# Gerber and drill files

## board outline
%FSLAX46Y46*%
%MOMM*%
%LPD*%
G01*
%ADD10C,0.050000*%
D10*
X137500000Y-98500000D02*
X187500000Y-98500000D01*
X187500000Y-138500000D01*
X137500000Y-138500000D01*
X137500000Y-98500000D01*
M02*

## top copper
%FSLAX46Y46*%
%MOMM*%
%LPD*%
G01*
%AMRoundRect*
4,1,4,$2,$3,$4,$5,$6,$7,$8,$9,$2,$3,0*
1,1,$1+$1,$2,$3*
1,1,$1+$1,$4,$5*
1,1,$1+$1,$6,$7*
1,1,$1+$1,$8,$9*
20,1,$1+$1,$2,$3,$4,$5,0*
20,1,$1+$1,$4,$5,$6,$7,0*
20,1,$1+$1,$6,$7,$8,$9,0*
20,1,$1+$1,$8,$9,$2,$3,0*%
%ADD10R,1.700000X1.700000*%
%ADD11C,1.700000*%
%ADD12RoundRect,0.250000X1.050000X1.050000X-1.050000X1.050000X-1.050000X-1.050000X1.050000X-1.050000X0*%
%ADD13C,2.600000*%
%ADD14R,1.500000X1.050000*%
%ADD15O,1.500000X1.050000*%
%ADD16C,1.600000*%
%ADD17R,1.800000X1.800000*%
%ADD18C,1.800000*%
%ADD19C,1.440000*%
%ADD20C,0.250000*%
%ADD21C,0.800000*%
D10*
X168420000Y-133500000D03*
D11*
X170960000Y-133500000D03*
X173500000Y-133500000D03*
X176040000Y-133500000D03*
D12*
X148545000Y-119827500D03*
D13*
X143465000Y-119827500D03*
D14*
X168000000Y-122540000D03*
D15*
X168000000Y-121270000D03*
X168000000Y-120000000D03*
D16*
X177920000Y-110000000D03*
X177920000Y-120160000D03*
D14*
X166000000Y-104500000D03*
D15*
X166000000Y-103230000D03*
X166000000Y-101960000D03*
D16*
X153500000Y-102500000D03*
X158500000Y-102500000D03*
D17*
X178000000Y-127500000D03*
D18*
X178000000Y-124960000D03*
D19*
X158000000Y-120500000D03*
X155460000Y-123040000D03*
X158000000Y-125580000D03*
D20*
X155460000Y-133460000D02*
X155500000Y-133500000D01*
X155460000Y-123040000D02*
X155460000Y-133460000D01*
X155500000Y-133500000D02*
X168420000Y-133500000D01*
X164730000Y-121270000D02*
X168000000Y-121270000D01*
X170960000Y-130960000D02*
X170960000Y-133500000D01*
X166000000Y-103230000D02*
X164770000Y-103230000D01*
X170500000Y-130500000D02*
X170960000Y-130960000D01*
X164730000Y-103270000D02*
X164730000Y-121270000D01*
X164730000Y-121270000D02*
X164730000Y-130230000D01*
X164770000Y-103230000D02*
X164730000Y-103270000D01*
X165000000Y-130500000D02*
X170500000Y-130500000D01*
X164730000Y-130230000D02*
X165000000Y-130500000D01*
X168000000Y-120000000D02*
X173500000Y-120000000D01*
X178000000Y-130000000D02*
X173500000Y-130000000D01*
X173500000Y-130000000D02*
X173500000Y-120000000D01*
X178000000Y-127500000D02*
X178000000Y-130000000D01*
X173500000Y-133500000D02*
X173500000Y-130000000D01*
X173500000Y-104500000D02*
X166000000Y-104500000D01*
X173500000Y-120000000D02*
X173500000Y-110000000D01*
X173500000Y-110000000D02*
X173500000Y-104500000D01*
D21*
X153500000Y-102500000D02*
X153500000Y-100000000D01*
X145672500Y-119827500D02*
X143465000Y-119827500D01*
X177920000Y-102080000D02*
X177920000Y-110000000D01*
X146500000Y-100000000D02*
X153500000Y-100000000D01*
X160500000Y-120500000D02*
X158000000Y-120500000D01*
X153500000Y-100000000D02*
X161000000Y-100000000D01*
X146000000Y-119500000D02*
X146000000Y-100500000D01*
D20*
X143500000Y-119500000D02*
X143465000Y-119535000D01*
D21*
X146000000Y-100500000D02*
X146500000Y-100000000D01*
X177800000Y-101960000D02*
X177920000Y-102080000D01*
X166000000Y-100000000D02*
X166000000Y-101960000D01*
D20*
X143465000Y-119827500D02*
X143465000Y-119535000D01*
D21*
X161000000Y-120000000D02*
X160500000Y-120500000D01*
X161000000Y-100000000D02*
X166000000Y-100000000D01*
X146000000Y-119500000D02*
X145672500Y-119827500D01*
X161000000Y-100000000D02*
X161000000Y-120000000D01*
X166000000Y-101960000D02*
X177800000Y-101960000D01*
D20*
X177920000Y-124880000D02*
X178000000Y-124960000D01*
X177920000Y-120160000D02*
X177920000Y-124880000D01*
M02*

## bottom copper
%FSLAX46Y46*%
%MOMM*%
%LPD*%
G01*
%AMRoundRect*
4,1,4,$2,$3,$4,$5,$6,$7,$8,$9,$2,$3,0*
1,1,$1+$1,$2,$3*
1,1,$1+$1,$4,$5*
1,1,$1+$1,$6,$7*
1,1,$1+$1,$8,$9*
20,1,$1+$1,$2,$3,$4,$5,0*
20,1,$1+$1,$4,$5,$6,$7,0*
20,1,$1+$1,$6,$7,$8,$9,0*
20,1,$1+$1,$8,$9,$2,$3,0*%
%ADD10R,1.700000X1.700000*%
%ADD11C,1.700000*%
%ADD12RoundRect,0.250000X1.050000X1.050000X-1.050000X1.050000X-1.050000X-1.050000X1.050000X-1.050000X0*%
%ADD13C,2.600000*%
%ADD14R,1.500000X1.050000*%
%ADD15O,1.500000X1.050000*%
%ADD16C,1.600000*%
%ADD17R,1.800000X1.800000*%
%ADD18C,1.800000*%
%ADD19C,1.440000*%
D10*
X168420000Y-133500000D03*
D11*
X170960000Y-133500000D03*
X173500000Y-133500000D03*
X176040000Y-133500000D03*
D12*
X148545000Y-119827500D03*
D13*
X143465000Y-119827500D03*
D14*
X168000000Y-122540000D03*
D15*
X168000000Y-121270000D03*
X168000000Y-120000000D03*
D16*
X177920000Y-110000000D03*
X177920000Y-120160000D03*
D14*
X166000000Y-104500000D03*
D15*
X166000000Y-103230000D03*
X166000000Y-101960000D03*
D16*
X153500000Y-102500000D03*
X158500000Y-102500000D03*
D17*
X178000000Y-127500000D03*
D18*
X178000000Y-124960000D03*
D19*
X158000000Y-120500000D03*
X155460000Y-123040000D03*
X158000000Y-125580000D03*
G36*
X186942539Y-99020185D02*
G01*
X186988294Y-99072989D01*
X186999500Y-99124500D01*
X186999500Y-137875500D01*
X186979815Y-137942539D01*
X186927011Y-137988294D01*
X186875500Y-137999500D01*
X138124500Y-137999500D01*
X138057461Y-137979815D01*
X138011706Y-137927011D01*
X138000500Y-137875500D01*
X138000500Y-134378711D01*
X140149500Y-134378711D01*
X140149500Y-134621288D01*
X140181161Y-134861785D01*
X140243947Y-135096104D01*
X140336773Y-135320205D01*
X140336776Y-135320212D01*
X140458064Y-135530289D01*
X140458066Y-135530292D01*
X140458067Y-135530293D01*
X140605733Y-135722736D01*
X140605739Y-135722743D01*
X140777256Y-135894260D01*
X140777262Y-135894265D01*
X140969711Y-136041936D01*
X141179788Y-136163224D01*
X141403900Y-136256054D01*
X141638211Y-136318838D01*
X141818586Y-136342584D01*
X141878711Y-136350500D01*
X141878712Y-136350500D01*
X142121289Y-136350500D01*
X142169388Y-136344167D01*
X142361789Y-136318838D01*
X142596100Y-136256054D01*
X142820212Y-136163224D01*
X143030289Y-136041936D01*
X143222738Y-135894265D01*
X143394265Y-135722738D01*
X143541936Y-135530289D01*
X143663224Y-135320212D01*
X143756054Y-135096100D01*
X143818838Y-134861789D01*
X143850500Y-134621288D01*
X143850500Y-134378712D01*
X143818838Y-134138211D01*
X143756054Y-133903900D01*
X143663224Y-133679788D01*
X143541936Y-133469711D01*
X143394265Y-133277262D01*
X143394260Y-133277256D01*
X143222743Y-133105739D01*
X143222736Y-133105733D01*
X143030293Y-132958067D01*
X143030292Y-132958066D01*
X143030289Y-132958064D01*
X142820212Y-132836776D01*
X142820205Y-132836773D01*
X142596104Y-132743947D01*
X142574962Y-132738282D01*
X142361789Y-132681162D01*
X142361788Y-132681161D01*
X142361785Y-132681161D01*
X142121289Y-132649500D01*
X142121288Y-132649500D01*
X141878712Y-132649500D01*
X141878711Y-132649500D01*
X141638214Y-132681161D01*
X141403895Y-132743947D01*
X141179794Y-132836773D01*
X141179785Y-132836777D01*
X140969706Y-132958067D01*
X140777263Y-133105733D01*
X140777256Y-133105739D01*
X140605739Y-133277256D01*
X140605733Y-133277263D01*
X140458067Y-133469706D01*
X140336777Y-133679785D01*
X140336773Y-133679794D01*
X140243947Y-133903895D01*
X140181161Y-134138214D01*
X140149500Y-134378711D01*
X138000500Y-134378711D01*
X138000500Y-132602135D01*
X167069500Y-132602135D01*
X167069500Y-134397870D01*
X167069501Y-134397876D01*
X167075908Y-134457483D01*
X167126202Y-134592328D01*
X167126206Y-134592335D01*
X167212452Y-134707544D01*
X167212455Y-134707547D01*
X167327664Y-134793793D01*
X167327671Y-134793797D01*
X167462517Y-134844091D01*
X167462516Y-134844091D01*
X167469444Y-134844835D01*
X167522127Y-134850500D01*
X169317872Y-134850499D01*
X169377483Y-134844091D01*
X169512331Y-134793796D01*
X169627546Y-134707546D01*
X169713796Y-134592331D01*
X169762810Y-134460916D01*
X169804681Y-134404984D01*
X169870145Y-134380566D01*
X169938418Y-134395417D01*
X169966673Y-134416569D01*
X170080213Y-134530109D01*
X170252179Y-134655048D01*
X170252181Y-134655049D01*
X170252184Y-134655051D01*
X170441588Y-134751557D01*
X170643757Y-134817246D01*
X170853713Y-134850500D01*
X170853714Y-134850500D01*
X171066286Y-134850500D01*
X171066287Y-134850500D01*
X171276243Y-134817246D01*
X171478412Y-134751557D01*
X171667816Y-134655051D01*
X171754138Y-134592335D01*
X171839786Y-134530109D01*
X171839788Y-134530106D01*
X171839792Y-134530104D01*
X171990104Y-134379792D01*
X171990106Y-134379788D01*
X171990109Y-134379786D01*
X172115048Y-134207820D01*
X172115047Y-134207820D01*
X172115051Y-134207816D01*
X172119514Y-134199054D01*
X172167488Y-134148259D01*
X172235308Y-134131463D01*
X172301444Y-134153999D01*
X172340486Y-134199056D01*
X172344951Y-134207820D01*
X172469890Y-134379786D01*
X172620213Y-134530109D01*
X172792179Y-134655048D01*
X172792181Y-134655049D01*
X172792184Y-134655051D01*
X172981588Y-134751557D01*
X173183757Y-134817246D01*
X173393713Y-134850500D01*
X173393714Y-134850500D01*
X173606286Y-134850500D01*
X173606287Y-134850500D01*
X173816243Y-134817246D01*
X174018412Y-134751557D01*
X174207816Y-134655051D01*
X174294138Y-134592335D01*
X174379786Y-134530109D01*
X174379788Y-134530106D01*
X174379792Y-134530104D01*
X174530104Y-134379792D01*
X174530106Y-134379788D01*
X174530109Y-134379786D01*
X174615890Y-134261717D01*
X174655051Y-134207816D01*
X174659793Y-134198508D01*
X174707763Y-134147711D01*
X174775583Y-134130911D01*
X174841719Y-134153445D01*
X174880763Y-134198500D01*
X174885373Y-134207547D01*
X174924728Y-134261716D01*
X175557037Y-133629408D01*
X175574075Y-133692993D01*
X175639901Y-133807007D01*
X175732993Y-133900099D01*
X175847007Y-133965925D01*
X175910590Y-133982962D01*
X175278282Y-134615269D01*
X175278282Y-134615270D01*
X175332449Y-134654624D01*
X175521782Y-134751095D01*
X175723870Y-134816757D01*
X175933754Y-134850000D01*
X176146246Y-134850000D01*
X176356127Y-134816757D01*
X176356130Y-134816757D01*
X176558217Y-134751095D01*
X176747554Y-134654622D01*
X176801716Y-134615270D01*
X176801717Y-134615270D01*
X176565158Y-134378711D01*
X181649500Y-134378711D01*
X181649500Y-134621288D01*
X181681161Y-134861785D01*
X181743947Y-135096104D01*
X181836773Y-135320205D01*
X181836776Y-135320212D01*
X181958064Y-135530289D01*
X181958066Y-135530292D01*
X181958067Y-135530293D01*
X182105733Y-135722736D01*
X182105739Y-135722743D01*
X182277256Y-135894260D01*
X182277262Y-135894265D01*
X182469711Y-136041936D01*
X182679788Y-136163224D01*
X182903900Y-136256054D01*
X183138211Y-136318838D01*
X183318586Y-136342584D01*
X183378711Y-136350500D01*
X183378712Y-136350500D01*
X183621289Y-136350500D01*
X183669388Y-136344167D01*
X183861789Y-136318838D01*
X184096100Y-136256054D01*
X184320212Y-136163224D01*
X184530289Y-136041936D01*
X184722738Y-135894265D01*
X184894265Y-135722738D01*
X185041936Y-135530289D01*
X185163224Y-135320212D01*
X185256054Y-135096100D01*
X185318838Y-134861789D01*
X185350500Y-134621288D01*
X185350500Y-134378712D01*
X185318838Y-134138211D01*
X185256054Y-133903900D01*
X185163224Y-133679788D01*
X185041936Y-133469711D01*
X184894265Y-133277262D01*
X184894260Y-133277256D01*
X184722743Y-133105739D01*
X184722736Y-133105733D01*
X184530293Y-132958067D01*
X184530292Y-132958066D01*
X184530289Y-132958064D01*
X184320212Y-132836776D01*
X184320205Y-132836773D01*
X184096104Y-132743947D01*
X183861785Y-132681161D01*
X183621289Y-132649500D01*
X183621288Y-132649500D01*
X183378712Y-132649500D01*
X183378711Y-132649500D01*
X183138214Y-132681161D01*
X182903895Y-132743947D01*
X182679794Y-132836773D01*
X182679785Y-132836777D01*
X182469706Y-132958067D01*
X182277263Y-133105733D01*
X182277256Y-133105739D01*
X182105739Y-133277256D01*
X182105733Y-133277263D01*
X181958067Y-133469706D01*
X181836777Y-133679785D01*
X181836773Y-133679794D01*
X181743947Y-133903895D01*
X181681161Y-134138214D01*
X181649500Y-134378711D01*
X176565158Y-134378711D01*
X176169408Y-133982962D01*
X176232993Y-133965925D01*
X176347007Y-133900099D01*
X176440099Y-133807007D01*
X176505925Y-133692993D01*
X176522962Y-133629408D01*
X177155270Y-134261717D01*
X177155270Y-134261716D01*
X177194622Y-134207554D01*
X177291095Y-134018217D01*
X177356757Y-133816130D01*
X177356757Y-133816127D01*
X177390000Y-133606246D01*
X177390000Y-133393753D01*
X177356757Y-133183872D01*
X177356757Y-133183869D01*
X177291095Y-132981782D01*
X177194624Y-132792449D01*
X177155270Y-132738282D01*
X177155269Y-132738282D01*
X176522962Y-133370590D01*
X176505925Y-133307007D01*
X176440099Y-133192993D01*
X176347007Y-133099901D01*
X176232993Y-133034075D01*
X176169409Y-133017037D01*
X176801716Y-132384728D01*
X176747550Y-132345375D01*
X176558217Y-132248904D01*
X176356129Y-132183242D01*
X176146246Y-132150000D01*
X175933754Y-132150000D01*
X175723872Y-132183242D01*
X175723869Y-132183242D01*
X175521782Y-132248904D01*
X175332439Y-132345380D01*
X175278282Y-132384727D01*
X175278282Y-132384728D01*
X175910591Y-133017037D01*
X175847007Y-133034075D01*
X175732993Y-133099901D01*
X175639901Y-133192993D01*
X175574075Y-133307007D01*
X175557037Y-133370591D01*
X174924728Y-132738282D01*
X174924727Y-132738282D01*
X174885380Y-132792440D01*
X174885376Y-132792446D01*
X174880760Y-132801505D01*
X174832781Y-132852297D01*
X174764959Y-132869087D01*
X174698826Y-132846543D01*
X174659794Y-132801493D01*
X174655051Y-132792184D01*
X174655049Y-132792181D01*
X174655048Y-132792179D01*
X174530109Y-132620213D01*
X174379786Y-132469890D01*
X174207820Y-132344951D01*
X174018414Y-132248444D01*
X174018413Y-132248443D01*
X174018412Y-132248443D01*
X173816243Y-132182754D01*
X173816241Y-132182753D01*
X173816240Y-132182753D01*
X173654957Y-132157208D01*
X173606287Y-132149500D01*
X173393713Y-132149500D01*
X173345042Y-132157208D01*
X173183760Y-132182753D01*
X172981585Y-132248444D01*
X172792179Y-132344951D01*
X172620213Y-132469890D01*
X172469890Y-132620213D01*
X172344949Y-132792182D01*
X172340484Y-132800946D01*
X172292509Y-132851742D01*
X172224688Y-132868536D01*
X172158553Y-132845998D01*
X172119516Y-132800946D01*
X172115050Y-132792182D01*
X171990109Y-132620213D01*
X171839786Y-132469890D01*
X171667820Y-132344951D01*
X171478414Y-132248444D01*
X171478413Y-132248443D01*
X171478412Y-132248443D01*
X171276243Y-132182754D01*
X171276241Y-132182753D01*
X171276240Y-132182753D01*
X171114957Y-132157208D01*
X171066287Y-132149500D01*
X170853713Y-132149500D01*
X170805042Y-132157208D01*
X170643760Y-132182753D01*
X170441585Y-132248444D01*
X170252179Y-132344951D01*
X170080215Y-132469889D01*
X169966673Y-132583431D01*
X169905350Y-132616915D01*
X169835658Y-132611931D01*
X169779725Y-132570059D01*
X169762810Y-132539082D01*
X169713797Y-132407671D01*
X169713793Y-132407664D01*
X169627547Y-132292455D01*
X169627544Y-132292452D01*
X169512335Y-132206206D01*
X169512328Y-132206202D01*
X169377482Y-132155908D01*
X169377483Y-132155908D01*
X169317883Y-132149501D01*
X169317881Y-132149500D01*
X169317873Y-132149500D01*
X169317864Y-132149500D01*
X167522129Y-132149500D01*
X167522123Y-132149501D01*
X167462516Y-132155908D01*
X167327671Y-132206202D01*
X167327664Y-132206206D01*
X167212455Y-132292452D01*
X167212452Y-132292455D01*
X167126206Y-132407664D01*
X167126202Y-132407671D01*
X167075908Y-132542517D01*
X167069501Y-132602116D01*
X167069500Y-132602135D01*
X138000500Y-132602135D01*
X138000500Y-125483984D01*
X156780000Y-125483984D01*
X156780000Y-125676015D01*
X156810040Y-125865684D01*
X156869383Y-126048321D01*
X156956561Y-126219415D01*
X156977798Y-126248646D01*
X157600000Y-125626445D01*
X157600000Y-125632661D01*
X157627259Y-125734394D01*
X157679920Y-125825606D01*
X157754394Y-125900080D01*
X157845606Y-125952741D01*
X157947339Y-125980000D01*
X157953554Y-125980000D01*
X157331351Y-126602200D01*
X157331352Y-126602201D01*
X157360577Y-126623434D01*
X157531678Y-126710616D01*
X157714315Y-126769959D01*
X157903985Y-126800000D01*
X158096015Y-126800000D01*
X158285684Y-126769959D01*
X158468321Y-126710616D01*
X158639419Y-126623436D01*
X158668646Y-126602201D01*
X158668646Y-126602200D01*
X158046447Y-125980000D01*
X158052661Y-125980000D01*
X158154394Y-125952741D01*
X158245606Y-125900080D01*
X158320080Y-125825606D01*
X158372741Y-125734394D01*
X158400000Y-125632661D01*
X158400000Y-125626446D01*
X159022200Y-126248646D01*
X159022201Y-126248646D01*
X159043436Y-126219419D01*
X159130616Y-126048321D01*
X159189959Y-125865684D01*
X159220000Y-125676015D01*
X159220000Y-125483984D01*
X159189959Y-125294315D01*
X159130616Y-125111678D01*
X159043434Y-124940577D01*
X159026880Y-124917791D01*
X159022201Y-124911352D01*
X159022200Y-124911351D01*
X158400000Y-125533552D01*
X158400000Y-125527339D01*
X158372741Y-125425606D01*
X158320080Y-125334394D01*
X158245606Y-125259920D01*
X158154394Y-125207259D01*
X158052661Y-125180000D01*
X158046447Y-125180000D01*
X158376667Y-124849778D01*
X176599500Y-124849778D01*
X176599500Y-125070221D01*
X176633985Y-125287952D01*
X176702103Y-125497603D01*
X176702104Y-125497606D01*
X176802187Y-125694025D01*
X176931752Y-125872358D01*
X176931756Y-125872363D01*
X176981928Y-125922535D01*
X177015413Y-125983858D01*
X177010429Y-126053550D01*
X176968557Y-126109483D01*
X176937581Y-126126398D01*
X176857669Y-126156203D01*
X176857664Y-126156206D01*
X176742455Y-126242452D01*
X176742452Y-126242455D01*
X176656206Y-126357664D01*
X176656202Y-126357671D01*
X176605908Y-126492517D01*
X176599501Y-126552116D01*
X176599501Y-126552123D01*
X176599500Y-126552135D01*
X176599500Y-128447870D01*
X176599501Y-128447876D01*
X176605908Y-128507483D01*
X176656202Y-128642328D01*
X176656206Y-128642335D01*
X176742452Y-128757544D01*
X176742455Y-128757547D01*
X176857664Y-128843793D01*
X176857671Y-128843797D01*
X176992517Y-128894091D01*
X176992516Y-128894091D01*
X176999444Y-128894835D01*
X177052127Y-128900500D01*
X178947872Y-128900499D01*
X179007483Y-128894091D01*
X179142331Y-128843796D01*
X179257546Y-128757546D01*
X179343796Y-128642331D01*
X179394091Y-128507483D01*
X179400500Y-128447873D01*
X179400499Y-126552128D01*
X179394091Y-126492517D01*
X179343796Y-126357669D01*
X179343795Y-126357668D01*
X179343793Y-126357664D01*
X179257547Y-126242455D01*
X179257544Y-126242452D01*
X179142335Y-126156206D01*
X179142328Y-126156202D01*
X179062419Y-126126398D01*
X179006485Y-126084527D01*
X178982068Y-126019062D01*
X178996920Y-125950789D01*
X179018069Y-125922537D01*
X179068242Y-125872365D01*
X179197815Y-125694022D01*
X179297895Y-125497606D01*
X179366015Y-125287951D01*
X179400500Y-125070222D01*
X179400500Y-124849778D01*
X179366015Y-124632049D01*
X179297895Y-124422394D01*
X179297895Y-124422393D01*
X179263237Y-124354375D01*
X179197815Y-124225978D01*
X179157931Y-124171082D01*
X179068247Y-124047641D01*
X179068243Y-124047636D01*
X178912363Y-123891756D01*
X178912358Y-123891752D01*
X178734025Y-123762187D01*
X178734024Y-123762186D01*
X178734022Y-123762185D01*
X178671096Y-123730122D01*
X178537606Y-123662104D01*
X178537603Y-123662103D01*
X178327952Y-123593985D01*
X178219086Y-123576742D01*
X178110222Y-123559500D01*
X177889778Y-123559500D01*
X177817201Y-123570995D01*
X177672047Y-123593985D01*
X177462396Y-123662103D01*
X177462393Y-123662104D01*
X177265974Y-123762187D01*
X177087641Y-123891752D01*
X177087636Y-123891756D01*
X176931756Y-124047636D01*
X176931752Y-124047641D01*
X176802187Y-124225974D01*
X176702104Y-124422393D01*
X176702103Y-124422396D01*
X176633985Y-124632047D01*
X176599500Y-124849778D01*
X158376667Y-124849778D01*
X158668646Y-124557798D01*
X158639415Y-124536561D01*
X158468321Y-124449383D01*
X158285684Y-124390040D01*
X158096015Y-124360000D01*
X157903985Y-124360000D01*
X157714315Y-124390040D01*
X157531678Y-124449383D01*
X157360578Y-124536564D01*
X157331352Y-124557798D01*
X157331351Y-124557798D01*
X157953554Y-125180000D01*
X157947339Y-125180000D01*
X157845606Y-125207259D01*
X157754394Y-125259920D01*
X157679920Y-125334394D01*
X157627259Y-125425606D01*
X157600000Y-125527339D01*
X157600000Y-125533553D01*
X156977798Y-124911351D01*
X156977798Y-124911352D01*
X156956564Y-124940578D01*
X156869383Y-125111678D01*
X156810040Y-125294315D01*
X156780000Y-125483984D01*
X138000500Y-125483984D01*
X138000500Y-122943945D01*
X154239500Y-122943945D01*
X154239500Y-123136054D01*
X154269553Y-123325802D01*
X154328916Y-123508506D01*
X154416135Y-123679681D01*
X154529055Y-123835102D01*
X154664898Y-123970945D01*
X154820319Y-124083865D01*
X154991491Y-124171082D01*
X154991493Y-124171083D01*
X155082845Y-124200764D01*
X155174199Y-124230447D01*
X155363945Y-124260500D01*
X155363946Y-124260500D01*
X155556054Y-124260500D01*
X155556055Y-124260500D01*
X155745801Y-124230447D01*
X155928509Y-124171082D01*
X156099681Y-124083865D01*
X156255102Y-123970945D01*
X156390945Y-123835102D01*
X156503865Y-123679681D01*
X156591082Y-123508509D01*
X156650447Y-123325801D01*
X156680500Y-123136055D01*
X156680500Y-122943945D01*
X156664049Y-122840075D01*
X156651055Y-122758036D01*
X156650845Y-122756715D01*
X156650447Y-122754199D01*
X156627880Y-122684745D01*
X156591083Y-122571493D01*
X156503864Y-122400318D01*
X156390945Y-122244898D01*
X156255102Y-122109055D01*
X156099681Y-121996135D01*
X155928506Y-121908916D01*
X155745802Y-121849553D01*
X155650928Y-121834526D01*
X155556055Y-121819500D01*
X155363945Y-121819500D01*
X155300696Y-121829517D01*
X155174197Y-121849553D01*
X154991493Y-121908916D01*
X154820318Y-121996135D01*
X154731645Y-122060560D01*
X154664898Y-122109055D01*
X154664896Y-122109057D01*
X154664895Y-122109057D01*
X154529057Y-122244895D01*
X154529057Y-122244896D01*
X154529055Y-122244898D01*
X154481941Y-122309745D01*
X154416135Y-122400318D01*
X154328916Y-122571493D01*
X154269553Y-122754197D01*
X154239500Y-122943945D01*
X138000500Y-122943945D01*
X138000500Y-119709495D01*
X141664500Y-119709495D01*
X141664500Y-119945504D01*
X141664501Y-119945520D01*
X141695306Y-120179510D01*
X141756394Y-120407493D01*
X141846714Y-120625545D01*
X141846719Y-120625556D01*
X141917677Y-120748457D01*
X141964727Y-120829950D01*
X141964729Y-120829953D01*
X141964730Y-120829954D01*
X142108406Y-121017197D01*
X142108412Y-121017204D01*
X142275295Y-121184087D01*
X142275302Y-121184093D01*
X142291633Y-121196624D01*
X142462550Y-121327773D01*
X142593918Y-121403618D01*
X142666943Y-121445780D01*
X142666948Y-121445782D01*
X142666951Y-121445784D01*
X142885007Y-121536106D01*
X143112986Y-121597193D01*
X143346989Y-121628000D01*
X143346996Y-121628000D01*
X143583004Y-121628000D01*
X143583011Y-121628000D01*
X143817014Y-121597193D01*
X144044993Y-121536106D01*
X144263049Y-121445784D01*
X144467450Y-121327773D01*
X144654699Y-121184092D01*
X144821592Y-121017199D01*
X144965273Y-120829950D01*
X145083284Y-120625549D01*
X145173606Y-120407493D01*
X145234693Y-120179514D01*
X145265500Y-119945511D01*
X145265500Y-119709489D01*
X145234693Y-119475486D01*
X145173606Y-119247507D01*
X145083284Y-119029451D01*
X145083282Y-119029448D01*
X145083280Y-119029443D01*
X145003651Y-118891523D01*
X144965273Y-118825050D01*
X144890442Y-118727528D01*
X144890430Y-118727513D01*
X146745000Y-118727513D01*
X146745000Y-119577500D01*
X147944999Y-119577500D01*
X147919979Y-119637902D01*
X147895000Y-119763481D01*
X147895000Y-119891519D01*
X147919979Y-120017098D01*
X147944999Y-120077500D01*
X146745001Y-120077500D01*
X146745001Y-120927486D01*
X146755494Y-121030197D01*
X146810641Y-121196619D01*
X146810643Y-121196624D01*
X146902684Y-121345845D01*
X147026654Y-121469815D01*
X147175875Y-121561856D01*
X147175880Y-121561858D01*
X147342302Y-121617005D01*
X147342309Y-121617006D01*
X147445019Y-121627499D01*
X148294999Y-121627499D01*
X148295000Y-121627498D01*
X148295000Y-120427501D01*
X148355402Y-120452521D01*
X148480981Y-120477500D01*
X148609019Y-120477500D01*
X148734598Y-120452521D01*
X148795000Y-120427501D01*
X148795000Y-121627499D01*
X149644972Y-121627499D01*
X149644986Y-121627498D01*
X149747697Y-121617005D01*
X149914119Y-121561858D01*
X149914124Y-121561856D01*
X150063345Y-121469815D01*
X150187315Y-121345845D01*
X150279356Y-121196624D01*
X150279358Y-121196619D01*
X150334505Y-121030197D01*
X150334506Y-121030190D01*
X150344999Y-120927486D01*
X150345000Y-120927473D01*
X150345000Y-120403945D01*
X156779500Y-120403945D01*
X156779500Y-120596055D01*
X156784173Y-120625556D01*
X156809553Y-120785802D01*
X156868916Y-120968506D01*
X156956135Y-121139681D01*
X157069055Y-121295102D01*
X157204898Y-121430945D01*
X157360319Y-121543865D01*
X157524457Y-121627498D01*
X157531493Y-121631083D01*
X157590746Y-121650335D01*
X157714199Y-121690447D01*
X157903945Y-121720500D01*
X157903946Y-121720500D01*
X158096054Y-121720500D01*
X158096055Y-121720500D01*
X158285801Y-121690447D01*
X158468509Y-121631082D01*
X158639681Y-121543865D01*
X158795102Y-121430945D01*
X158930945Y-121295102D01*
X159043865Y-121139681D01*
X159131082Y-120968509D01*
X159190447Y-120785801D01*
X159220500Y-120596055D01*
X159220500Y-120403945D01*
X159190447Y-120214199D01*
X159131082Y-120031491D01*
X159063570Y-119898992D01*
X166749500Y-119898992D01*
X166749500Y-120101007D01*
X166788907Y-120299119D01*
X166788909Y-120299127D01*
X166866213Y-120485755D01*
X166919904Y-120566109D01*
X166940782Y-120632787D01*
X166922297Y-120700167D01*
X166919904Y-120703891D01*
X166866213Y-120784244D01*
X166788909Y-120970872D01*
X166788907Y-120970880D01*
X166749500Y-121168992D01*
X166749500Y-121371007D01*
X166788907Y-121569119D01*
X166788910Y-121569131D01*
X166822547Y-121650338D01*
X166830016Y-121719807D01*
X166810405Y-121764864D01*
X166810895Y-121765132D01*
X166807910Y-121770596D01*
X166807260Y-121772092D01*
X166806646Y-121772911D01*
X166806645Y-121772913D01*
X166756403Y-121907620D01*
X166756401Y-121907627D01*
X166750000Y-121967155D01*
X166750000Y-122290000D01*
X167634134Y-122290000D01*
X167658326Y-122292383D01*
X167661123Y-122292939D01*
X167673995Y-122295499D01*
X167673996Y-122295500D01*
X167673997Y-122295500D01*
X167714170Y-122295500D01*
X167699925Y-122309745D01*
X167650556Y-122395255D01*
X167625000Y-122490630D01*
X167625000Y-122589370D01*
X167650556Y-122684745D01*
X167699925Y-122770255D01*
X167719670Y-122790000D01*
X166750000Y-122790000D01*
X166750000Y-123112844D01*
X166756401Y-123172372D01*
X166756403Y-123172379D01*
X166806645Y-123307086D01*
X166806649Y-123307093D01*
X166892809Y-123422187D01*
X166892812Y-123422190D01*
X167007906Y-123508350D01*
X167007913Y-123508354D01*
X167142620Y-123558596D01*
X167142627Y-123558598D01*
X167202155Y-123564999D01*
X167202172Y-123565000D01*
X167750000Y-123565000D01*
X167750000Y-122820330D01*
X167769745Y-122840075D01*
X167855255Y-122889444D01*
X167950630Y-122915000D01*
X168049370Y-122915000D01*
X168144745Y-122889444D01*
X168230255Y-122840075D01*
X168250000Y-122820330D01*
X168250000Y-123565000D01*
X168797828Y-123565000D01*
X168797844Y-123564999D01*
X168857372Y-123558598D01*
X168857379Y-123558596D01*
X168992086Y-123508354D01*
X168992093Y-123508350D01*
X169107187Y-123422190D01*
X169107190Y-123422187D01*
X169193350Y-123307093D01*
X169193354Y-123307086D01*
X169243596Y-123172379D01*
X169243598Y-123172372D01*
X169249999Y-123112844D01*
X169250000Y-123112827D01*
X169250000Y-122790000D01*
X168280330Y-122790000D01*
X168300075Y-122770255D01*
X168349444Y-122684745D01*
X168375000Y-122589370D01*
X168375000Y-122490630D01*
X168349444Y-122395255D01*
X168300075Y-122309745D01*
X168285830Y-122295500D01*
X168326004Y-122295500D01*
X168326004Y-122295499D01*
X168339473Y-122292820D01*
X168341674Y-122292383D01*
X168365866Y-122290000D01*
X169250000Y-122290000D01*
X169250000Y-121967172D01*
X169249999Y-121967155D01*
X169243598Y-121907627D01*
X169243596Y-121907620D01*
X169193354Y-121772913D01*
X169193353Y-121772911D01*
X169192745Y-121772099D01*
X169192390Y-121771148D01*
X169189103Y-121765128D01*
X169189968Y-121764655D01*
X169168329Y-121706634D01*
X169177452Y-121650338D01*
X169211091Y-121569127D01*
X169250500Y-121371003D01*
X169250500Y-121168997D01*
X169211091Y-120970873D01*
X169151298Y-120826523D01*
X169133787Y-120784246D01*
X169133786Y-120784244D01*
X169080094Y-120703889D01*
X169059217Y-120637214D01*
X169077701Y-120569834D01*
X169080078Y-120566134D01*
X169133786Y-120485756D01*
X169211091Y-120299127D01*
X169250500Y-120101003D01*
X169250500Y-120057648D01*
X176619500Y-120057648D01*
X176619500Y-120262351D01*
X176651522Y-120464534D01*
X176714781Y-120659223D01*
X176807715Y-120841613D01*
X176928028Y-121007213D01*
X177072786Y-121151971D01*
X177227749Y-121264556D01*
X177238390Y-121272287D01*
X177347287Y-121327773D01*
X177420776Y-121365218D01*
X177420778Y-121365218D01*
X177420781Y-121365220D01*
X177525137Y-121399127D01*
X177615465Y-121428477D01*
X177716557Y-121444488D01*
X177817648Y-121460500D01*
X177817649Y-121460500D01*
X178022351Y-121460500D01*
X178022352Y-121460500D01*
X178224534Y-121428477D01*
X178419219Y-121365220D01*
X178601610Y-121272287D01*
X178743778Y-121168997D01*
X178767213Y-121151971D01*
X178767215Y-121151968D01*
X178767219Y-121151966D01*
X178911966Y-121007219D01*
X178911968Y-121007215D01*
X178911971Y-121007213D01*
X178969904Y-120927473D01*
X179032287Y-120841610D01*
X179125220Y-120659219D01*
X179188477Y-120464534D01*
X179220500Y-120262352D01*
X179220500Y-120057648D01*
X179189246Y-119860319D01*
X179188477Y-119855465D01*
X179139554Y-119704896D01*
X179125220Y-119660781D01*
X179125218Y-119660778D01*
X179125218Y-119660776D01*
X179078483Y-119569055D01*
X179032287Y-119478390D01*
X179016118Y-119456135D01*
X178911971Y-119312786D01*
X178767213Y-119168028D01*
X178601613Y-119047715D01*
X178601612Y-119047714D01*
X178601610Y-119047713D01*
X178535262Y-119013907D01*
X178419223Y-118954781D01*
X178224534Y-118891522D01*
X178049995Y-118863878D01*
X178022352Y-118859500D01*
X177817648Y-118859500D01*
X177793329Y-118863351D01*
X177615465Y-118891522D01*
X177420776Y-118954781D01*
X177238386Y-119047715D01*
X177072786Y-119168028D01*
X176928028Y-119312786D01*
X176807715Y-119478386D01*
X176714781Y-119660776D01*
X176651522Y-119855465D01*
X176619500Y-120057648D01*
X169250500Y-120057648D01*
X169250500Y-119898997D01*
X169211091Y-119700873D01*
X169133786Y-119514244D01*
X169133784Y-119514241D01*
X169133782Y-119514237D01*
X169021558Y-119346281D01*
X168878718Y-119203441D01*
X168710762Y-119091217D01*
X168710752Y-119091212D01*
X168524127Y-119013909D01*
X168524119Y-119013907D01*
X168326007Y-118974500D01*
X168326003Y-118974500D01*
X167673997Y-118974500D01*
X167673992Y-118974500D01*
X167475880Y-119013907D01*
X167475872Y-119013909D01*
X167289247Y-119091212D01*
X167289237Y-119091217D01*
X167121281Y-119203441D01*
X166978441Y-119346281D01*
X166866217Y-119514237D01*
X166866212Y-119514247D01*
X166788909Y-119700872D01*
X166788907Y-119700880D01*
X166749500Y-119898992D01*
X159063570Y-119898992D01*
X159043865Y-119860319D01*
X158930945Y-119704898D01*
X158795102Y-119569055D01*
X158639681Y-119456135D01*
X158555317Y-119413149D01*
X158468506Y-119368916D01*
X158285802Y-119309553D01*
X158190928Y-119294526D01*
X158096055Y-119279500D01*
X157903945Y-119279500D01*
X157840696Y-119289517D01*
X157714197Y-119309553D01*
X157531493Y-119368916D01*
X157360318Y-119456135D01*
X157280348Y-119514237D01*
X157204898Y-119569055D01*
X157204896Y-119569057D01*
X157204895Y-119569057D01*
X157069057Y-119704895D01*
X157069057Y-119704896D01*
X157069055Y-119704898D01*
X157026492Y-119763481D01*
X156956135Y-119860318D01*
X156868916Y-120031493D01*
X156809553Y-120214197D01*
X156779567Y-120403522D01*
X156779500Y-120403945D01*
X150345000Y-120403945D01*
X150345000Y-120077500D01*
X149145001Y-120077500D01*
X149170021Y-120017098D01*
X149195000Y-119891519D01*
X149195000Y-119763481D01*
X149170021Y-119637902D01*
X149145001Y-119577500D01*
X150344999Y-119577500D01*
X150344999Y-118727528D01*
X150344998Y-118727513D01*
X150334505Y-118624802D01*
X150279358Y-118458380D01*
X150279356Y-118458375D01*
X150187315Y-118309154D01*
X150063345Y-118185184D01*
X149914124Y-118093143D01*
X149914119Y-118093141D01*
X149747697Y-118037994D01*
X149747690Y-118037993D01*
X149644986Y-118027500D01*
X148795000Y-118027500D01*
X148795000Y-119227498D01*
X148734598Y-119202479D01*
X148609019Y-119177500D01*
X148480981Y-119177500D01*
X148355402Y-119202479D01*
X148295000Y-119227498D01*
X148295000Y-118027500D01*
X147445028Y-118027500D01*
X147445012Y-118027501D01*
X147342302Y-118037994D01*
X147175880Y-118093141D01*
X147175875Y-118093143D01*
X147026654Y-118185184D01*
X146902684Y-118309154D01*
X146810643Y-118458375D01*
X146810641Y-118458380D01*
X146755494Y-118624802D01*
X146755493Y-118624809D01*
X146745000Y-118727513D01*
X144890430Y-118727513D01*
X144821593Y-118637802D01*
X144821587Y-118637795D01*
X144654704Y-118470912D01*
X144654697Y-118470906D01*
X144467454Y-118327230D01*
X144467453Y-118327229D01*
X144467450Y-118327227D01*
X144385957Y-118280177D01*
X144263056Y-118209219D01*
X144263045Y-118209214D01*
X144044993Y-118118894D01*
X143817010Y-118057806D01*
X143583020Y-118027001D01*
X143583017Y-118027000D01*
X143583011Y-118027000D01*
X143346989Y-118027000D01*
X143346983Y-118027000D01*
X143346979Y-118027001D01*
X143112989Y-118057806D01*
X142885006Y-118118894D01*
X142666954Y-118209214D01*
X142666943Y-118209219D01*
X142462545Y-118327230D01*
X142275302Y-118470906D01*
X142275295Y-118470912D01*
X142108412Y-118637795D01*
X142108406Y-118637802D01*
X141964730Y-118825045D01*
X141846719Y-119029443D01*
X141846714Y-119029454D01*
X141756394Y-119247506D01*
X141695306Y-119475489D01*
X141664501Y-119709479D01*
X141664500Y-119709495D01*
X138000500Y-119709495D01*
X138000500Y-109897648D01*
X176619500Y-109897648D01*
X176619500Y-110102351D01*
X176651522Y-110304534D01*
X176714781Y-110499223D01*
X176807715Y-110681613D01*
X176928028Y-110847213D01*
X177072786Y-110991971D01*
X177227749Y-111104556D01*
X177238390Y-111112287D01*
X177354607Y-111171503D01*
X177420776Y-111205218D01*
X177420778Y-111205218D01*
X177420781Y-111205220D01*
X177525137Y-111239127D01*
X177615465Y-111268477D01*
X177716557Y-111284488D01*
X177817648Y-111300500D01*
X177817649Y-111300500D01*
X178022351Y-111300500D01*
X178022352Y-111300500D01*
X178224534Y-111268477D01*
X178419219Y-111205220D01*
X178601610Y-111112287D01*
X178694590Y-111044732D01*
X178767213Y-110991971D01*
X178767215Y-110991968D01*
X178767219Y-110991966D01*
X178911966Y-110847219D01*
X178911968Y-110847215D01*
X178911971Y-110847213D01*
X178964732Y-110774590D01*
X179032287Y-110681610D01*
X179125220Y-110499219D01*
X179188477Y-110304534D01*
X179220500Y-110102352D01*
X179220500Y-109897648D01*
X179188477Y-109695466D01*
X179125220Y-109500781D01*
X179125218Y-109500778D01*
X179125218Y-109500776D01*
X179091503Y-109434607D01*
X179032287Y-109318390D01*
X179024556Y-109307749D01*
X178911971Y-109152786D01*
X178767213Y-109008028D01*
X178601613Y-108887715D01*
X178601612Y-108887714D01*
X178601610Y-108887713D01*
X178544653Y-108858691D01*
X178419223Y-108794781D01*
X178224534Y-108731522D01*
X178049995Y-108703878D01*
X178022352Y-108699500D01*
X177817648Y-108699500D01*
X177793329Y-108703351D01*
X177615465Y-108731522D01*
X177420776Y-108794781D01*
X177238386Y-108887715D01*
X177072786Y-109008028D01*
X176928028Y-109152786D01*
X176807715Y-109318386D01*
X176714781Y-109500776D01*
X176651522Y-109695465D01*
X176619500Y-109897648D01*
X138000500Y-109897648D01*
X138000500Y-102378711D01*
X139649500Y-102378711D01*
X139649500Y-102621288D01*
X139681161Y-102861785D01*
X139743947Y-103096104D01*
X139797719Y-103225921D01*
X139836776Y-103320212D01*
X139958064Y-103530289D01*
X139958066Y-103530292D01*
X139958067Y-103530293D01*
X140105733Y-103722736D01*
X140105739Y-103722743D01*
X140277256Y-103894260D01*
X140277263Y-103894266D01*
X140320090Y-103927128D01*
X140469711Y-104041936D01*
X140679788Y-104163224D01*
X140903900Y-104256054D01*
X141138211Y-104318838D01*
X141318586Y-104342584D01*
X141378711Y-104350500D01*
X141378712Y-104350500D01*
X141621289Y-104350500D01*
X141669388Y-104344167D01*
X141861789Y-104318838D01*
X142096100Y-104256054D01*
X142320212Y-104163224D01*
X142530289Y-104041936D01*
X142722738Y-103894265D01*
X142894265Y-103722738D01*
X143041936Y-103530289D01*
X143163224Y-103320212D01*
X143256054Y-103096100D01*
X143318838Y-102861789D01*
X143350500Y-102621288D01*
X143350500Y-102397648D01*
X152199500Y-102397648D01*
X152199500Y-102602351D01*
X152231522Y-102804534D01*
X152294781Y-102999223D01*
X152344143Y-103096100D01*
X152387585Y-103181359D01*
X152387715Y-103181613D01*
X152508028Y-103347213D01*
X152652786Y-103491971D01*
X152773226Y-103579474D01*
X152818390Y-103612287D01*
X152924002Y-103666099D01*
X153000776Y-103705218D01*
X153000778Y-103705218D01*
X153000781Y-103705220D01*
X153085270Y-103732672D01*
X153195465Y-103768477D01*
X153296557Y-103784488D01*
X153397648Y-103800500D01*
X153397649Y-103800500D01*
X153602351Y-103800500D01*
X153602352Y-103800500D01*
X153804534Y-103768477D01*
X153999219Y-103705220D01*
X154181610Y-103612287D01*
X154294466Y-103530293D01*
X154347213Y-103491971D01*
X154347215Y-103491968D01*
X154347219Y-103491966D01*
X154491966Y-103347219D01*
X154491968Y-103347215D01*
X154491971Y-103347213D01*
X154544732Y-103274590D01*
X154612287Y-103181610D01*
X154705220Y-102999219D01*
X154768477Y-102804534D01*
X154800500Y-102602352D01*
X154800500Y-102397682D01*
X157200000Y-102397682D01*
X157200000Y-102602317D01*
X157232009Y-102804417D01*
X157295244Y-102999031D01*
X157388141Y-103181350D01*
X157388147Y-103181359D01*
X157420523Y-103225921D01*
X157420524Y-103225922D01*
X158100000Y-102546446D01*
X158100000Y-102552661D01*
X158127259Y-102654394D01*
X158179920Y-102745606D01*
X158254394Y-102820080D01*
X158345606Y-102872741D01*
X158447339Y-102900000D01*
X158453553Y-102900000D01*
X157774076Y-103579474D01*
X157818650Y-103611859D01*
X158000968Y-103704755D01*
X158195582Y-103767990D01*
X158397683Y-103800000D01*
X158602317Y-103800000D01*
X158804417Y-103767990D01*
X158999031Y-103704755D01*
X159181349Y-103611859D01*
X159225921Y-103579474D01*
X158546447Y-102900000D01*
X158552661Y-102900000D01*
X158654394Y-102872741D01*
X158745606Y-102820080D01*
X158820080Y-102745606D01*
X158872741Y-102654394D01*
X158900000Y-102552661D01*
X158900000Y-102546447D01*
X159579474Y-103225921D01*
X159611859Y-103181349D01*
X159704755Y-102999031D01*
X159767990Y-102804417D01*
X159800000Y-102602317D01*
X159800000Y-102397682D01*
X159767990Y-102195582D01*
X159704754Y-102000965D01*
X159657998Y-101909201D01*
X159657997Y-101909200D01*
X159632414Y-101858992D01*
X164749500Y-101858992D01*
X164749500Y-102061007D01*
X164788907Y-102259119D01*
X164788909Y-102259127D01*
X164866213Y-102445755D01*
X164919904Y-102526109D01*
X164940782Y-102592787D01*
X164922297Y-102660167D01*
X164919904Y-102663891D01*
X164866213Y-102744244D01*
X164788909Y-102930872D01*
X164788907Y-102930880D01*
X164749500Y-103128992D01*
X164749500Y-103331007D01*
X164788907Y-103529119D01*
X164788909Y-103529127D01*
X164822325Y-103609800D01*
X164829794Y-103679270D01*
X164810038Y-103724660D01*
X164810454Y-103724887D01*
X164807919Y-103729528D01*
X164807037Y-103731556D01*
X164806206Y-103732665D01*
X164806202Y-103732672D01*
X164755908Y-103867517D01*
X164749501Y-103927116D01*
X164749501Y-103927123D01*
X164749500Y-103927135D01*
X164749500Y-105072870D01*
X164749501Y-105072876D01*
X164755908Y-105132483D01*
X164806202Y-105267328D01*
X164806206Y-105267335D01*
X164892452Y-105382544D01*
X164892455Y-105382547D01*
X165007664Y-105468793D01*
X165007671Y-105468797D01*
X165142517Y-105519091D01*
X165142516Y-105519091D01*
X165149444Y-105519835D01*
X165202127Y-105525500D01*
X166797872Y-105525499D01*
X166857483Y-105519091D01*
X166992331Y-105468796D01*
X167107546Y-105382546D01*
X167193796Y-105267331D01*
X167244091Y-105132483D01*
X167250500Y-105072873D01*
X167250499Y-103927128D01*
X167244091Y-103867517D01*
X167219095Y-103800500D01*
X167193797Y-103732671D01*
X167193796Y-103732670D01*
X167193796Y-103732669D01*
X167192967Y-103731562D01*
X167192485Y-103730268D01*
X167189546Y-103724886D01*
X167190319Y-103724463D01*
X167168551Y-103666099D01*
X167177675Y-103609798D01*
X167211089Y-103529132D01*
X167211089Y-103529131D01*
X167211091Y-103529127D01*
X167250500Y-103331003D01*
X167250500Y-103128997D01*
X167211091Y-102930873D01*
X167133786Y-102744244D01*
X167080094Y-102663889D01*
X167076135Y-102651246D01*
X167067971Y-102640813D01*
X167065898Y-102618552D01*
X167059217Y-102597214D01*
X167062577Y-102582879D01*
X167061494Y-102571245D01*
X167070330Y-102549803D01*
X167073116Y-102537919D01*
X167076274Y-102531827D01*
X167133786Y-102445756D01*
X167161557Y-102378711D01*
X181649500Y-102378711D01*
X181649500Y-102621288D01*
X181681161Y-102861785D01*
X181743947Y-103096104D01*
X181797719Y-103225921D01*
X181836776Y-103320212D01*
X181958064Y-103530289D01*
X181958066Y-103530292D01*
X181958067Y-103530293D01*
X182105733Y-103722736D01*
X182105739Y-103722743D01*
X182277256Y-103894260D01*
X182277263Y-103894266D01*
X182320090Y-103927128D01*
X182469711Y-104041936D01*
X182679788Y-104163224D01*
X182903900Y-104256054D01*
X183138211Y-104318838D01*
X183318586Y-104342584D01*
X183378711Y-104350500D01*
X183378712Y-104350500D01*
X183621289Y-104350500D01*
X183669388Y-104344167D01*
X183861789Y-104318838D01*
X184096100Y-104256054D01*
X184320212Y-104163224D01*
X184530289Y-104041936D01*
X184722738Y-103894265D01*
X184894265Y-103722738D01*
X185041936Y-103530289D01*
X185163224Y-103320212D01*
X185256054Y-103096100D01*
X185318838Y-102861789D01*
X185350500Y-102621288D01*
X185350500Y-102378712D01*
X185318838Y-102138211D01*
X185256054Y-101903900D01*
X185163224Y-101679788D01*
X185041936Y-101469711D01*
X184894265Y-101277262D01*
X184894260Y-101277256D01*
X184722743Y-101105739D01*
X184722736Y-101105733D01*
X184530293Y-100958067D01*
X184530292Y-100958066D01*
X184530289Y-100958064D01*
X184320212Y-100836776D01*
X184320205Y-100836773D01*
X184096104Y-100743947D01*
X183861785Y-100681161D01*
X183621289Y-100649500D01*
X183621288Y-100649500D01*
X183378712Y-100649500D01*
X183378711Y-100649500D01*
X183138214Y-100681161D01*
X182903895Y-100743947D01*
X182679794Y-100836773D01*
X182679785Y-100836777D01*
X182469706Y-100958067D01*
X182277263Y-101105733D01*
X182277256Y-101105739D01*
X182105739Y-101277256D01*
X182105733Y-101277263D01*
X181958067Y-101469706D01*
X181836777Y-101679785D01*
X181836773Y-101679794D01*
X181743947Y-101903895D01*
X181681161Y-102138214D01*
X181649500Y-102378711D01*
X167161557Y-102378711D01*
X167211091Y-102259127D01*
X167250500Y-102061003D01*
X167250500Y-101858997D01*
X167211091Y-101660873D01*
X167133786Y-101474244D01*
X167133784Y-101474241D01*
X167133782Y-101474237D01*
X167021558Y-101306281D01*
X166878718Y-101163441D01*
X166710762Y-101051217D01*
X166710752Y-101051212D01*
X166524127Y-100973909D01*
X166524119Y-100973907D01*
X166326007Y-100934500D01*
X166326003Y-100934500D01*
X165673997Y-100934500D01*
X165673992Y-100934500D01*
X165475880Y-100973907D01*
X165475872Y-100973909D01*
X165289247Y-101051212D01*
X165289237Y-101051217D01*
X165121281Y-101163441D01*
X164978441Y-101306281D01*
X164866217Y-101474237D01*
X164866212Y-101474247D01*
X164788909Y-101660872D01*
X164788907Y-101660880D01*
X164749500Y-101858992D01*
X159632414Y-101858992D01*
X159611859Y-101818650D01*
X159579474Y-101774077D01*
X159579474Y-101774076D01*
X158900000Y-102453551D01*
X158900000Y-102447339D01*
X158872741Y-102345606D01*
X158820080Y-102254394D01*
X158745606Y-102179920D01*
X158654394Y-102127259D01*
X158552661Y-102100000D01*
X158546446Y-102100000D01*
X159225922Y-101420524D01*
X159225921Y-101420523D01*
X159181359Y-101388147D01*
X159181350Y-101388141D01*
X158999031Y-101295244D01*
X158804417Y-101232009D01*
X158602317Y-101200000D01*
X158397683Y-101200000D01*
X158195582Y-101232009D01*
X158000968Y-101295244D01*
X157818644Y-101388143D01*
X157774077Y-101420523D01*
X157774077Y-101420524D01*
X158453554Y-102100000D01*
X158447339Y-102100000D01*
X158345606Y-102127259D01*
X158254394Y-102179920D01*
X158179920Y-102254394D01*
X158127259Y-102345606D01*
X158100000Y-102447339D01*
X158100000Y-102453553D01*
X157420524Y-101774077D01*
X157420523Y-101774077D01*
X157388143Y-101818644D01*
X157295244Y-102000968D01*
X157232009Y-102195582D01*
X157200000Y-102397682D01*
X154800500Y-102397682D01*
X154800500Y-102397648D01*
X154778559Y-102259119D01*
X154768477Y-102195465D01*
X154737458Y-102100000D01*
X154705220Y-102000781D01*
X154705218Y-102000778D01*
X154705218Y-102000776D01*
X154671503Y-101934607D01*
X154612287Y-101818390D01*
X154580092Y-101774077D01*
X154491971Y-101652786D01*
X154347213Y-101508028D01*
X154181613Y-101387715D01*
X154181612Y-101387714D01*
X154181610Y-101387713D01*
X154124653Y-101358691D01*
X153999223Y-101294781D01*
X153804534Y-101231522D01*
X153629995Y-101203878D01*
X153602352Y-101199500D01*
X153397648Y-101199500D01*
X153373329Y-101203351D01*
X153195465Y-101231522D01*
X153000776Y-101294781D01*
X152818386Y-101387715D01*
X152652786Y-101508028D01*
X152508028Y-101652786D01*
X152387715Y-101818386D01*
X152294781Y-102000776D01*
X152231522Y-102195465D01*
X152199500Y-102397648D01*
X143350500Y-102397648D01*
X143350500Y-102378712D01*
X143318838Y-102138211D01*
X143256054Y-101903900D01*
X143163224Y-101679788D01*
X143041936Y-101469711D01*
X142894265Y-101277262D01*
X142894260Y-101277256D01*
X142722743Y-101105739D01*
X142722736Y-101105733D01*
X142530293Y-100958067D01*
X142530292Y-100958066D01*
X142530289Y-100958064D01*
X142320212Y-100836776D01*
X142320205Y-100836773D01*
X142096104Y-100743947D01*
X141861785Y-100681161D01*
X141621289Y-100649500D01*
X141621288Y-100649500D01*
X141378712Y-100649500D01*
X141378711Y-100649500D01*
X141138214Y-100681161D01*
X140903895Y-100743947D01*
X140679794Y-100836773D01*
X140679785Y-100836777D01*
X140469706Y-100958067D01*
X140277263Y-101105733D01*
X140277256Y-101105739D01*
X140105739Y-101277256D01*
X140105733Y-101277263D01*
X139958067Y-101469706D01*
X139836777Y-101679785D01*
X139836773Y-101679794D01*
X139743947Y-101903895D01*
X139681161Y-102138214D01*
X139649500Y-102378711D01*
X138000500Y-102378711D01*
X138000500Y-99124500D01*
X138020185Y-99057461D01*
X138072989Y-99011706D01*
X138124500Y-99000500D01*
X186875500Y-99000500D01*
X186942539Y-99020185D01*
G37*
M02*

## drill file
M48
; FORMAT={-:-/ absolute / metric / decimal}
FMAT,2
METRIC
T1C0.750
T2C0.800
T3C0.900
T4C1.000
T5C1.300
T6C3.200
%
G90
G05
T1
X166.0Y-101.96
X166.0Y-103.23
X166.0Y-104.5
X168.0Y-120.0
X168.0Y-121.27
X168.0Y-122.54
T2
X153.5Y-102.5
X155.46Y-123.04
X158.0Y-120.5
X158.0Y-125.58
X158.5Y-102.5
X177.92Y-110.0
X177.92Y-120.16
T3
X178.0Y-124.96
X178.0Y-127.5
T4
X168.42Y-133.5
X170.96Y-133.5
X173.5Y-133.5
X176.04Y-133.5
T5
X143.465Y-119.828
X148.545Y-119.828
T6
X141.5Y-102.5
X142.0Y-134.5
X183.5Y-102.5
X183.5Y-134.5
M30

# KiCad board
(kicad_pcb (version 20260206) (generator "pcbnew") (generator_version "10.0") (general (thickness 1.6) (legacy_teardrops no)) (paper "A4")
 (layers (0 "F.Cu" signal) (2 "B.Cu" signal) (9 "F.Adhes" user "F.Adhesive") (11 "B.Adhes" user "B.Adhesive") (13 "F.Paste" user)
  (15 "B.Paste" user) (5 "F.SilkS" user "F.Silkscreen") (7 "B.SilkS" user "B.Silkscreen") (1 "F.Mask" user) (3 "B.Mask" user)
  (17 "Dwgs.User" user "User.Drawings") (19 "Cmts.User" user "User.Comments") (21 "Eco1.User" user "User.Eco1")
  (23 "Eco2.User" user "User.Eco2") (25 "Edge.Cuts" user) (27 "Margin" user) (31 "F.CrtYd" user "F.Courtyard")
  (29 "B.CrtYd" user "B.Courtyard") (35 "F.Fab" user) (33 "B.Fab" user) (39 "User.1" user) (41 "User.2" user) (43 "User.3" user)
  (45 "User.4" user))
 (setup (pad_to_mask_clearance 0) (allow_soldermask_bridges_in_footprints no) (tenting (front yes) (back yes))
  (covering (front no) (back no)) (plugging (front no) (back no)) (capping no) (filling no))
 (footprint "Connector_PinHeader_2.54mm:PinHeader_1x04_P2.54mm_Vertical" (layer "F.Cu") (at 168.42 133.5 90)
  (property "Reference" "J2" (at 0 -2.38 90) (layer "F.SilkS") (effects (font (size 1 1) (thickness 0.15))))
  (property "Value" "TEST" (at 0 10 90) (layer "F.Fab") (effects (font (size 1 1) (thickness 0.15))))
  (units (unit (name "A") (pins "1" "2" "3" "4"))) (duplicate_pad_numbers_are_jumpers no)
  (pad "1" thru_hole rect (at 0 0 90) (size 1.7 1.7) (drill 1) (layers "*.Cu" "*.Mask") (remove_unused_layers no) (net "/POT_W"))
  (pad "2" thru_hole circle (at 0 2.54 90) (size 1.7 1.7) (drill 1) (layers "*.Cu" "*.Mask") (remove_unused_layers no) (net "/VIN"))
  (pad "3" thru_hole circle (at 0 5.08 90) (size 1.7 1.7) (drill 1) (layers "*.Cu" "*.Mask") (remove_unused_layers no) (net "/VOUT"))
  (pad "4" thru_hole circle (at 0 7.62 90) (size 1.7 1.7) (drill 1) (layers "*.Cu" "*.Mask") (remove_unused_layers no) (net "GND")))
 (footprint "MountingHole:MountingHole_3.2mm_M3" (layer "F.Cu") (at 141.5 102.5)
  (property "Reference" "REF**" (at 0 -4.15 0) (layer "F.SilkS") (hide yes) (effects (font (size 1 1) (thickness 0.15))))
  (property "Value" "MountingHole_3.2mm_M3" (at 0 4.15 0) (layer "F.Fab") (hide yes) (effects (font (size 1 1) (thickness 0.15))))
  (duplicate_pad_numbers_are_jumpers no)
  (pad "" np_thru_hole circle (at 0 0) (size 3.2 3.2) (drill 3.2) (layers "*.Cu" "*.Mask")))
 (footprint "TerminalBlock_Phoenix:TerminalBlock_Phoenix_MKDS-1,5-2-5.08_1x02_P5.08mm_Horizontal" (layer "F.Cu") (at 148.545 119.8275 180)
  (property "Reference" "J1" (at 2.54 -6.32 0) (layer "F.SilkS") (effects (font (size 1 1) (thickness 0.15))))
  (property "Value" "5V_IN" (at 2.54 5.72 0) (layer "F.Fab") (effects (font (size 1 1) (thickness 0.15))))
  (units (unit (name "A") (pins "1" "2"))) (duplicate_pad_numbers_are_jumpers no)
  (pad "1" thru_hole roundrect (at 0 0 180) (size 2.6 2.6) (drill 1.3) (layers "*.Cu" "*.Mask") (remove_unused_layers no)
   (roundrect_rratio 0.096154) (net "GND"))
  (pad "2" thru_hole circle (at 5.08 0 180) (size 2.6 2.6) (drill 1.3) (layers "*.Cu" "*.Mask") (remove_unused_layers no) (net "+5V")))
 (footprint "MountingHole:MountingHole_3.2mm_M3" (layer "F.Cu") (at 183.5 102.5)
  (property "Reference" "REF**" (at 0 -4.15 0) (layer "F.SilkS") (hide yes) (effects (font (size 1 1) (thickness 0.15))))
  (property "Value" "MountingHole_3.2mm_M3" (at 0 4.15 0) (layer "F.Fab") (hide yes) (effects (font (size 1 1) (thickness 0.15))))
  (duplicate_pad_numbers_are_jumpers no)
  (pad "" np_thru_hole circle (at 0 0) (size 3.2 3.2) (drill 3.2) (layers "*.Cu" "*.Mask")))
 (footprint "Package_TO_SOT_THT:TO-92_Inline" (layer "F.Cu") (at 168 122.54 90)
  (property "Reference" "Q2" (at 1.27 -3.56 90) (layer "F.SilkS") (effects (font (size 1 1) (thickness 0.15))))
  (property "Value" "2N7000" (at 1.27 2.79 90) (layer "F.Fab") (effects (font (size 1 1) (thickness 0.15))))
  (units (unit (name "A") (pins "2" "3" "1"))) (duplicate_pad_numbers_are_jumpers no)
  (pad "1" thru_hole rect (at 0 0 90) (size 1.05 1.5) (drill 0.75) (layers "*.Cu" "*.Mask") (remove_unused_layers no) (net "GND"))
  (pad "2" thru_hole oval (at 1.27 0 90) (size 1.05 1.5) (drill 0.75) (layers "*.Cu" "*.Mask") (remove_unused_layers no) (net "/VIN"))
  (pad "3" thru_hole oval (at 2.54 0 90) (size 1.05 1.5) (drill 0.75) (layers "*.Cu" "*.Mask") (remove_unused_layers no) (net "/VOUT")))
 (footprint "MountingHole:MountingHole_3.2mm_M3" (layer "F.Cu") (at 142 134.5)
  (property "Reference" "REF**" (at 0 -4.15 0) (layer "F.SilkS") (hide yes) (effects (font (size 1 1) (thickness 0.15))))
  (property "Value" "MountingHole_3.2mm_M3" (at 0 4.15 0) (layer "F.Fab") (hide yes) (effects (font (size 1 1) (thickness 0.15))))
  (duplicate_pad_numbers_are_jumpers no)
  (pad "" np_thru_hole circle (at 0 0) (size 3.2 3.2) (drill 3.2) (layers "*.Cu" "*.Mask")))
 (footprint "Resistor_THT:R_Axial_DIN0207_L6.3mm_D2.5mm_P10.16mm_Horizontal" (layer "F.Cu") (at 177.92 110 -90)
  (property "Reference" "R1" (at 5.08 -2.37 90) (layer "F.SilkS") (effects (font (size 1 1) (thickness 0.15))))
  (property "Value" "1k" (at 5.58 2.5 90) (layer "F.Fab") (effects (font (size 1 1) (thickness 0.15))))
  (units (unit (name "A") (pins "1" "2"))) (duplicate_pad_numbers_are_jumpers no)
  (pad "1" thru_hole circle (at 0 0 270) (size 1.6 1.6) (drill 0.8) (layers "*.Cu" "*.Mask") (remove_unused_layers no) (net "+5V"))
  (pad "2" thru_hole circle (at 10.16 0 270) (size 1.6 1.6) (drill 0.8) (layers "*.Cu" "*.Mask") (remove_unused_layers no)
   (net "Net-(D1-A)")))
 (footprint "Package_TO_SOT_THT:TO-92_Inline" (layer "F.Cu") (at 166 104.5 90)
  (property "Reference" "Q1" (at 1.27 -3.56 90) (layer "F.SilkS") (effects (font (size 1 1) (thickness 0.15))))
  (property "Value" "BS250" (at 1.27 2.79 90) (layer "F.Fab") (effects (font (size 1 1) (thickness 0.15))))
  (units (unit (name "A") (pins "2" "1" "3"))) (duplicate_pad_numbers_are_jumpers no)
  (pad "1" thru_hole rect (at 0 0 90) (size 1.05 1.5) (drill 0.75) (layers "*.Cu" "*.Mask") (remove_unused_layers no) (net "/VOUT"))
  (pad "2" thru_hole oval (at 1.27 0 90) (size 1.05 1.5) (drill 0.75) (layers "*.Cu" "*.Mask") (remove_unused_layers no) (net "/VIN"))
  (pad "3" thru_hole oval (at 2.54 0 90) (size 1.05 1.5) (drill 0.75) (layers "*.Cu" "*.Mask") (remove_unused_layers no) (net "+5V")))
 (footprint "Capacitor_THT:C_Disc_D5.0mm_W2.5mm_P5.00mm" (layer "F.Cu") (at 153.5 102.5)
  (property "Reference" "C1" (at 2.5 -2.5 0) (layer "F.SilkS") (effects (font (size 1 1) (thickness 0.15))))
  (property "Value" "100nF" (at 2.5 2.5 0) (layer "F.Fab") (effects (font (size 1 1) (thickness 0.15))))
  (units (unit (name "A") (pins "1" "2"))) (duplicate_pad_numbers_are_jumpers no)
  (pad "1" thru_hole circle (at 0 0) (size 1.6 1.6) (drill 0.8) (layers "*.Cu" "*.Mask") (remove_unused_layers no) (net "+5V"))
  (pad "2" thru_hole circle (at 5 0) (size 1.6 1.6) (drill 0.8) (layers "*.Cu" "*.Mask") (remove_unused_layers no) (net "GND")))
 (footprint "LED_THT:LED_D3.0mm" (layer "F.Cu") (at 178 127.5 90)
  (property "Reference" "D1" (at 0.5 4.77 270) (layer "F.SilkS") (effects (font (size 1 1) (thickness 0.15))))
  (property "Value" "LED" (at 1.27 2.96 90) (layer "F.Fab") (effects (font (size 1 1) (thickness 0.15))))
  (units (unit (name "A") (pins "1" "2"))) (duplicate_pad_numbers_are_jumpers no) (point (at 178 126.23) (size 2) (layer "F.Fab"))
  (pad "1" thru_hole rect (at 0 0 90) (size 1.8 1.8) (drill 0.9) (layers "*.Cu" "*.Mask") (remove_unused_layers no) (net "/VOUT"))
  (pad "2" thru_hole circle (at 2.54 0 90) (size 1.8 1.8) (drill 0.9) (layers "*.Cu" "*.Mask") (remove_unused_layers no) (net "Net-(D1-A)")))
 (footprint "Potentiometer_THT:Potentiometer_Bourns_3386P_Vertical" (layer "F.Cu") (at 158 120.5 180)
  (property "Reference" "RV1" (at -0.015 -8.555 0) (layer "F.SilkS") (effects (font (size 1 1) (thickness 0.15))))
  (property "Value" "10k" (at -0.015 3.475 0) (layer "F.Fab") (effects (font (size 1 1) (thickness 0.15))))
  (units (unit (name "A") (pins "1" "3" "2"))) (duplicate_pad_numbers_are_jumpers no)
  (pad "1" thru_hole circle (at 0 0 180) (size 1.44 1.44) (drill 0.8) (layers "*.Cu" "*.Mask") (remove_unused_layers no) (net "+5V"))
  (pad "2" thru_hole circle (at 2.54 -2.54 180) (size 1.44 1.44) (drill 0.8) (layers "*.Cu" "*.Mask") (remove_unused_layers no)
   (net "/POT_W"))
  (pad "3" thru_hole circle (at 0 -5.08 180) (size 1.44 1.44) (drill 0.8) (layers "*.Cu" "*.Mask") (remove_unused_layers no) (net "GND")))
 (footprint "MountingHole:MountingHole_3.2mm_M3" (layer "F.Cu") (at 183.5 134.5)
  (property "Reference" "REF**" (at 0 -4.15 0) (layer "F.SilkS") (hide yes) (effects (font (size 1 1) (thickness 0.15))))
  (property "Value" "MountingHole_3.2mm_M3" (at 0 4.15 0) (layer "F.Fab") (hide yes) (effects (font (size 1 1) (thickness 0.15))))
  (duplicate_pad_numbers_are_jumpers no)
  (pad "" np_thru_hole circle (at 0 0) (size 3.2 3.2) (drill 3.2) (layers "*.Cu" "*.Mask")))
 (gr_rect (start 137.5 98.5) (end 187.5 138.5) (stroke (width 0.05) (type default)) (fill no) (layer "Edge.Cuts"))
 (segment (start 155.46 133.46) (end 155.5 133.5) (width 0.25) (layer "F.Cu") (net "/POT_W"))
 (segment (start 155.46 123.04) (end 155.46 133.46) (width 0.25) (layer "F.Cu") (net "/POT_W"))
 (segment (start 155.5 133.5) (end 168.42 133.5) (width 0.25) (layer "F.Cu") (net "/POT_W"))
 (segment (start 164.73 121.27) (end 168 121.27) (width 0.25) (layer "F.Cu") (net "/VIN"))
 (segment (start 170.96 130.96) (end 170.96 133.5) (width 0.25) (layer "F.Cu") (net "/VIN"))
 (segment (start 166 103.23) (end 164.77 103.23) (width 0.25) (layer "F.Cu") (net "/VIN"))
 (segment (start 170.5 130.5) (end 170.96 130.96) (width 0.25) (layer "F.Cu") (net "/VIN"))
 (segment (start 164.73 103.27) (end 164.73 121.27) (width 0.25) (layer "F.Cu") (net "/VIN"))
 (segment (start 164.73 121.27) (end 164.73 130.23) (width 0.25) (layer "F.Cu") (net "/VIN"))
 (segment (start 164.77 103.23) (end 164.73 103.27) (width 0.25) (layer "F.Cu") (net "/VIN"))
 (segment (start 165 130.5) (end 170.5 130.5) (width 0.25) (layer "F.Cu") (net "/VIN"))
 (segment (start 164.73 130.23) (end 165 130.5) (width 0.25) (layer "F.Cu") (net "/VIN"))
 (segment (start 168 120) (end 173.5 120) (width 0.25) (layer "F.Cu") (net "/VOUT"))
 (segment (start 178 130) (end 173.5 130) (width 0.25) (layer "F.Cu") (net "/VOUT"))
 (segment (start 173.5 130) (end 173.5 120) (width 0.25) (layer "F.Cu") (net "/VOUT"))
 (segment (start 178 127.5) (end 178 130) (width 0.25) (layer "F.Cu") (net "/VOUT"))
 (segment (start 173.5 133.5) (end 173.5 130) (width 0.25) (layer "F.Cu") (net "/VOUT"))
 (segment (start 173.5 104.5) (end 166 104.5) (width 0.25) (layer "F.Cu") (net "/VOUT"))
 (segment (start 173.5 120) (end 173.5 110) (width 0.25) (layer "F.Cu") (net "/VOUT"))
 (segment (start 173.5 110) (end 173.5 104.5) (width 0.25) (layer "F.Cu") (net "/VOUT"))
 (segment (start 153.5 102.5) (end 153.5 100) (width 0.8) (layer "F.Cu") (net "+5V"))
 (segment (start 145.6725 119.8275) (end 143.465 119.8275) (width 0.8) (layer "F.Cu") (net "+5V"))
 (segment (start 177.92 102.08) (end 177.92 110) (width 0.8) (layer "F.Cu") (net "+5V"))
 (segment (start 146.5 100) (end 153.5 100) (width 0.8) (layer "F.Cu") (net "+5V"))
 (segment (start 160.5 120.5) (end 158 120.5) (width 0.8) (layer "F.Cu") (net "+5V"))
 (segment (start 153.5 100) (end 161 100) (width 0.8) (layer "F.Cu") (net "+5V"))
 (segment (start 146 119.5) (end 146 100.5) (width 0.8) (layer "F.Cu") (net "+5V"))
 (segment (start 143.5 119.5) (end 143.465 119.535) (width 0.25) (layer "F.Cu") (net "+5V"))
 (segment (start 146 100.5) (end 146.5 100) (width 0.8) (layer "F.Cu") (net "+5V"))
 (segment (start 177.8 101.96) (end 177.92 102.08) (width 0.8) (layer "F.Cu") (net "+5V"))
 (segment (start 166 100) (end 166 101.96) (width 0.8) (layer "F.Cu") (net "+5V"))
 (segment (start 143.465 119.8275) (end 143.465 119.535) (width 0.25) (layer "F.Cu") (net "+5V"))
 (segment (start 161 120) (end 160.5 120.5) (width 0.8) (layer "F.Cu") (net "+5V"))
 (segment (start 161 100) (end 166 100) (width 0.8) (layer "F.Cu") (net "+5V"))
 (segment (start 146 119.5) (end 145.6725 119.8275) (width 0.8) (layer "F.Cu") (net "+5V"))
 (segment (start 161 100) (end 161 120) (width 0.8) (layer "F.Cu") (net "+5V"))
 (segment (start 166 101.96) (end 177.8 101.96) (width 0.8) (layer "F.Cu") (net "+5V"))
 (segment (start 177.92 124.88) (end 178 124.96) (width 0.25) (layer "F.Cu") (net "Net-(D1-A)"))
 (segment (start 177.92 120.16) (end 177.92 124.88) (width 0.25) (layer "F.Cu") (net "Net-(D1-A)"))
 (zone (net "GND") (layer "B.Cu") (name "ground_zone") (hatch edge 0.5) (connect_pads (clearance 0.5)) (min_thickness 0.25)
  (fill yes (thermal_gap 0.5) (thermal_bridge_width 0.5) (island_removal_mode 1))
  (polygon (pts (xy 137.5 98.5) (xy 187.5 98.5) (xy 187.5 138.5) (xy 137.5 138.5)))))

